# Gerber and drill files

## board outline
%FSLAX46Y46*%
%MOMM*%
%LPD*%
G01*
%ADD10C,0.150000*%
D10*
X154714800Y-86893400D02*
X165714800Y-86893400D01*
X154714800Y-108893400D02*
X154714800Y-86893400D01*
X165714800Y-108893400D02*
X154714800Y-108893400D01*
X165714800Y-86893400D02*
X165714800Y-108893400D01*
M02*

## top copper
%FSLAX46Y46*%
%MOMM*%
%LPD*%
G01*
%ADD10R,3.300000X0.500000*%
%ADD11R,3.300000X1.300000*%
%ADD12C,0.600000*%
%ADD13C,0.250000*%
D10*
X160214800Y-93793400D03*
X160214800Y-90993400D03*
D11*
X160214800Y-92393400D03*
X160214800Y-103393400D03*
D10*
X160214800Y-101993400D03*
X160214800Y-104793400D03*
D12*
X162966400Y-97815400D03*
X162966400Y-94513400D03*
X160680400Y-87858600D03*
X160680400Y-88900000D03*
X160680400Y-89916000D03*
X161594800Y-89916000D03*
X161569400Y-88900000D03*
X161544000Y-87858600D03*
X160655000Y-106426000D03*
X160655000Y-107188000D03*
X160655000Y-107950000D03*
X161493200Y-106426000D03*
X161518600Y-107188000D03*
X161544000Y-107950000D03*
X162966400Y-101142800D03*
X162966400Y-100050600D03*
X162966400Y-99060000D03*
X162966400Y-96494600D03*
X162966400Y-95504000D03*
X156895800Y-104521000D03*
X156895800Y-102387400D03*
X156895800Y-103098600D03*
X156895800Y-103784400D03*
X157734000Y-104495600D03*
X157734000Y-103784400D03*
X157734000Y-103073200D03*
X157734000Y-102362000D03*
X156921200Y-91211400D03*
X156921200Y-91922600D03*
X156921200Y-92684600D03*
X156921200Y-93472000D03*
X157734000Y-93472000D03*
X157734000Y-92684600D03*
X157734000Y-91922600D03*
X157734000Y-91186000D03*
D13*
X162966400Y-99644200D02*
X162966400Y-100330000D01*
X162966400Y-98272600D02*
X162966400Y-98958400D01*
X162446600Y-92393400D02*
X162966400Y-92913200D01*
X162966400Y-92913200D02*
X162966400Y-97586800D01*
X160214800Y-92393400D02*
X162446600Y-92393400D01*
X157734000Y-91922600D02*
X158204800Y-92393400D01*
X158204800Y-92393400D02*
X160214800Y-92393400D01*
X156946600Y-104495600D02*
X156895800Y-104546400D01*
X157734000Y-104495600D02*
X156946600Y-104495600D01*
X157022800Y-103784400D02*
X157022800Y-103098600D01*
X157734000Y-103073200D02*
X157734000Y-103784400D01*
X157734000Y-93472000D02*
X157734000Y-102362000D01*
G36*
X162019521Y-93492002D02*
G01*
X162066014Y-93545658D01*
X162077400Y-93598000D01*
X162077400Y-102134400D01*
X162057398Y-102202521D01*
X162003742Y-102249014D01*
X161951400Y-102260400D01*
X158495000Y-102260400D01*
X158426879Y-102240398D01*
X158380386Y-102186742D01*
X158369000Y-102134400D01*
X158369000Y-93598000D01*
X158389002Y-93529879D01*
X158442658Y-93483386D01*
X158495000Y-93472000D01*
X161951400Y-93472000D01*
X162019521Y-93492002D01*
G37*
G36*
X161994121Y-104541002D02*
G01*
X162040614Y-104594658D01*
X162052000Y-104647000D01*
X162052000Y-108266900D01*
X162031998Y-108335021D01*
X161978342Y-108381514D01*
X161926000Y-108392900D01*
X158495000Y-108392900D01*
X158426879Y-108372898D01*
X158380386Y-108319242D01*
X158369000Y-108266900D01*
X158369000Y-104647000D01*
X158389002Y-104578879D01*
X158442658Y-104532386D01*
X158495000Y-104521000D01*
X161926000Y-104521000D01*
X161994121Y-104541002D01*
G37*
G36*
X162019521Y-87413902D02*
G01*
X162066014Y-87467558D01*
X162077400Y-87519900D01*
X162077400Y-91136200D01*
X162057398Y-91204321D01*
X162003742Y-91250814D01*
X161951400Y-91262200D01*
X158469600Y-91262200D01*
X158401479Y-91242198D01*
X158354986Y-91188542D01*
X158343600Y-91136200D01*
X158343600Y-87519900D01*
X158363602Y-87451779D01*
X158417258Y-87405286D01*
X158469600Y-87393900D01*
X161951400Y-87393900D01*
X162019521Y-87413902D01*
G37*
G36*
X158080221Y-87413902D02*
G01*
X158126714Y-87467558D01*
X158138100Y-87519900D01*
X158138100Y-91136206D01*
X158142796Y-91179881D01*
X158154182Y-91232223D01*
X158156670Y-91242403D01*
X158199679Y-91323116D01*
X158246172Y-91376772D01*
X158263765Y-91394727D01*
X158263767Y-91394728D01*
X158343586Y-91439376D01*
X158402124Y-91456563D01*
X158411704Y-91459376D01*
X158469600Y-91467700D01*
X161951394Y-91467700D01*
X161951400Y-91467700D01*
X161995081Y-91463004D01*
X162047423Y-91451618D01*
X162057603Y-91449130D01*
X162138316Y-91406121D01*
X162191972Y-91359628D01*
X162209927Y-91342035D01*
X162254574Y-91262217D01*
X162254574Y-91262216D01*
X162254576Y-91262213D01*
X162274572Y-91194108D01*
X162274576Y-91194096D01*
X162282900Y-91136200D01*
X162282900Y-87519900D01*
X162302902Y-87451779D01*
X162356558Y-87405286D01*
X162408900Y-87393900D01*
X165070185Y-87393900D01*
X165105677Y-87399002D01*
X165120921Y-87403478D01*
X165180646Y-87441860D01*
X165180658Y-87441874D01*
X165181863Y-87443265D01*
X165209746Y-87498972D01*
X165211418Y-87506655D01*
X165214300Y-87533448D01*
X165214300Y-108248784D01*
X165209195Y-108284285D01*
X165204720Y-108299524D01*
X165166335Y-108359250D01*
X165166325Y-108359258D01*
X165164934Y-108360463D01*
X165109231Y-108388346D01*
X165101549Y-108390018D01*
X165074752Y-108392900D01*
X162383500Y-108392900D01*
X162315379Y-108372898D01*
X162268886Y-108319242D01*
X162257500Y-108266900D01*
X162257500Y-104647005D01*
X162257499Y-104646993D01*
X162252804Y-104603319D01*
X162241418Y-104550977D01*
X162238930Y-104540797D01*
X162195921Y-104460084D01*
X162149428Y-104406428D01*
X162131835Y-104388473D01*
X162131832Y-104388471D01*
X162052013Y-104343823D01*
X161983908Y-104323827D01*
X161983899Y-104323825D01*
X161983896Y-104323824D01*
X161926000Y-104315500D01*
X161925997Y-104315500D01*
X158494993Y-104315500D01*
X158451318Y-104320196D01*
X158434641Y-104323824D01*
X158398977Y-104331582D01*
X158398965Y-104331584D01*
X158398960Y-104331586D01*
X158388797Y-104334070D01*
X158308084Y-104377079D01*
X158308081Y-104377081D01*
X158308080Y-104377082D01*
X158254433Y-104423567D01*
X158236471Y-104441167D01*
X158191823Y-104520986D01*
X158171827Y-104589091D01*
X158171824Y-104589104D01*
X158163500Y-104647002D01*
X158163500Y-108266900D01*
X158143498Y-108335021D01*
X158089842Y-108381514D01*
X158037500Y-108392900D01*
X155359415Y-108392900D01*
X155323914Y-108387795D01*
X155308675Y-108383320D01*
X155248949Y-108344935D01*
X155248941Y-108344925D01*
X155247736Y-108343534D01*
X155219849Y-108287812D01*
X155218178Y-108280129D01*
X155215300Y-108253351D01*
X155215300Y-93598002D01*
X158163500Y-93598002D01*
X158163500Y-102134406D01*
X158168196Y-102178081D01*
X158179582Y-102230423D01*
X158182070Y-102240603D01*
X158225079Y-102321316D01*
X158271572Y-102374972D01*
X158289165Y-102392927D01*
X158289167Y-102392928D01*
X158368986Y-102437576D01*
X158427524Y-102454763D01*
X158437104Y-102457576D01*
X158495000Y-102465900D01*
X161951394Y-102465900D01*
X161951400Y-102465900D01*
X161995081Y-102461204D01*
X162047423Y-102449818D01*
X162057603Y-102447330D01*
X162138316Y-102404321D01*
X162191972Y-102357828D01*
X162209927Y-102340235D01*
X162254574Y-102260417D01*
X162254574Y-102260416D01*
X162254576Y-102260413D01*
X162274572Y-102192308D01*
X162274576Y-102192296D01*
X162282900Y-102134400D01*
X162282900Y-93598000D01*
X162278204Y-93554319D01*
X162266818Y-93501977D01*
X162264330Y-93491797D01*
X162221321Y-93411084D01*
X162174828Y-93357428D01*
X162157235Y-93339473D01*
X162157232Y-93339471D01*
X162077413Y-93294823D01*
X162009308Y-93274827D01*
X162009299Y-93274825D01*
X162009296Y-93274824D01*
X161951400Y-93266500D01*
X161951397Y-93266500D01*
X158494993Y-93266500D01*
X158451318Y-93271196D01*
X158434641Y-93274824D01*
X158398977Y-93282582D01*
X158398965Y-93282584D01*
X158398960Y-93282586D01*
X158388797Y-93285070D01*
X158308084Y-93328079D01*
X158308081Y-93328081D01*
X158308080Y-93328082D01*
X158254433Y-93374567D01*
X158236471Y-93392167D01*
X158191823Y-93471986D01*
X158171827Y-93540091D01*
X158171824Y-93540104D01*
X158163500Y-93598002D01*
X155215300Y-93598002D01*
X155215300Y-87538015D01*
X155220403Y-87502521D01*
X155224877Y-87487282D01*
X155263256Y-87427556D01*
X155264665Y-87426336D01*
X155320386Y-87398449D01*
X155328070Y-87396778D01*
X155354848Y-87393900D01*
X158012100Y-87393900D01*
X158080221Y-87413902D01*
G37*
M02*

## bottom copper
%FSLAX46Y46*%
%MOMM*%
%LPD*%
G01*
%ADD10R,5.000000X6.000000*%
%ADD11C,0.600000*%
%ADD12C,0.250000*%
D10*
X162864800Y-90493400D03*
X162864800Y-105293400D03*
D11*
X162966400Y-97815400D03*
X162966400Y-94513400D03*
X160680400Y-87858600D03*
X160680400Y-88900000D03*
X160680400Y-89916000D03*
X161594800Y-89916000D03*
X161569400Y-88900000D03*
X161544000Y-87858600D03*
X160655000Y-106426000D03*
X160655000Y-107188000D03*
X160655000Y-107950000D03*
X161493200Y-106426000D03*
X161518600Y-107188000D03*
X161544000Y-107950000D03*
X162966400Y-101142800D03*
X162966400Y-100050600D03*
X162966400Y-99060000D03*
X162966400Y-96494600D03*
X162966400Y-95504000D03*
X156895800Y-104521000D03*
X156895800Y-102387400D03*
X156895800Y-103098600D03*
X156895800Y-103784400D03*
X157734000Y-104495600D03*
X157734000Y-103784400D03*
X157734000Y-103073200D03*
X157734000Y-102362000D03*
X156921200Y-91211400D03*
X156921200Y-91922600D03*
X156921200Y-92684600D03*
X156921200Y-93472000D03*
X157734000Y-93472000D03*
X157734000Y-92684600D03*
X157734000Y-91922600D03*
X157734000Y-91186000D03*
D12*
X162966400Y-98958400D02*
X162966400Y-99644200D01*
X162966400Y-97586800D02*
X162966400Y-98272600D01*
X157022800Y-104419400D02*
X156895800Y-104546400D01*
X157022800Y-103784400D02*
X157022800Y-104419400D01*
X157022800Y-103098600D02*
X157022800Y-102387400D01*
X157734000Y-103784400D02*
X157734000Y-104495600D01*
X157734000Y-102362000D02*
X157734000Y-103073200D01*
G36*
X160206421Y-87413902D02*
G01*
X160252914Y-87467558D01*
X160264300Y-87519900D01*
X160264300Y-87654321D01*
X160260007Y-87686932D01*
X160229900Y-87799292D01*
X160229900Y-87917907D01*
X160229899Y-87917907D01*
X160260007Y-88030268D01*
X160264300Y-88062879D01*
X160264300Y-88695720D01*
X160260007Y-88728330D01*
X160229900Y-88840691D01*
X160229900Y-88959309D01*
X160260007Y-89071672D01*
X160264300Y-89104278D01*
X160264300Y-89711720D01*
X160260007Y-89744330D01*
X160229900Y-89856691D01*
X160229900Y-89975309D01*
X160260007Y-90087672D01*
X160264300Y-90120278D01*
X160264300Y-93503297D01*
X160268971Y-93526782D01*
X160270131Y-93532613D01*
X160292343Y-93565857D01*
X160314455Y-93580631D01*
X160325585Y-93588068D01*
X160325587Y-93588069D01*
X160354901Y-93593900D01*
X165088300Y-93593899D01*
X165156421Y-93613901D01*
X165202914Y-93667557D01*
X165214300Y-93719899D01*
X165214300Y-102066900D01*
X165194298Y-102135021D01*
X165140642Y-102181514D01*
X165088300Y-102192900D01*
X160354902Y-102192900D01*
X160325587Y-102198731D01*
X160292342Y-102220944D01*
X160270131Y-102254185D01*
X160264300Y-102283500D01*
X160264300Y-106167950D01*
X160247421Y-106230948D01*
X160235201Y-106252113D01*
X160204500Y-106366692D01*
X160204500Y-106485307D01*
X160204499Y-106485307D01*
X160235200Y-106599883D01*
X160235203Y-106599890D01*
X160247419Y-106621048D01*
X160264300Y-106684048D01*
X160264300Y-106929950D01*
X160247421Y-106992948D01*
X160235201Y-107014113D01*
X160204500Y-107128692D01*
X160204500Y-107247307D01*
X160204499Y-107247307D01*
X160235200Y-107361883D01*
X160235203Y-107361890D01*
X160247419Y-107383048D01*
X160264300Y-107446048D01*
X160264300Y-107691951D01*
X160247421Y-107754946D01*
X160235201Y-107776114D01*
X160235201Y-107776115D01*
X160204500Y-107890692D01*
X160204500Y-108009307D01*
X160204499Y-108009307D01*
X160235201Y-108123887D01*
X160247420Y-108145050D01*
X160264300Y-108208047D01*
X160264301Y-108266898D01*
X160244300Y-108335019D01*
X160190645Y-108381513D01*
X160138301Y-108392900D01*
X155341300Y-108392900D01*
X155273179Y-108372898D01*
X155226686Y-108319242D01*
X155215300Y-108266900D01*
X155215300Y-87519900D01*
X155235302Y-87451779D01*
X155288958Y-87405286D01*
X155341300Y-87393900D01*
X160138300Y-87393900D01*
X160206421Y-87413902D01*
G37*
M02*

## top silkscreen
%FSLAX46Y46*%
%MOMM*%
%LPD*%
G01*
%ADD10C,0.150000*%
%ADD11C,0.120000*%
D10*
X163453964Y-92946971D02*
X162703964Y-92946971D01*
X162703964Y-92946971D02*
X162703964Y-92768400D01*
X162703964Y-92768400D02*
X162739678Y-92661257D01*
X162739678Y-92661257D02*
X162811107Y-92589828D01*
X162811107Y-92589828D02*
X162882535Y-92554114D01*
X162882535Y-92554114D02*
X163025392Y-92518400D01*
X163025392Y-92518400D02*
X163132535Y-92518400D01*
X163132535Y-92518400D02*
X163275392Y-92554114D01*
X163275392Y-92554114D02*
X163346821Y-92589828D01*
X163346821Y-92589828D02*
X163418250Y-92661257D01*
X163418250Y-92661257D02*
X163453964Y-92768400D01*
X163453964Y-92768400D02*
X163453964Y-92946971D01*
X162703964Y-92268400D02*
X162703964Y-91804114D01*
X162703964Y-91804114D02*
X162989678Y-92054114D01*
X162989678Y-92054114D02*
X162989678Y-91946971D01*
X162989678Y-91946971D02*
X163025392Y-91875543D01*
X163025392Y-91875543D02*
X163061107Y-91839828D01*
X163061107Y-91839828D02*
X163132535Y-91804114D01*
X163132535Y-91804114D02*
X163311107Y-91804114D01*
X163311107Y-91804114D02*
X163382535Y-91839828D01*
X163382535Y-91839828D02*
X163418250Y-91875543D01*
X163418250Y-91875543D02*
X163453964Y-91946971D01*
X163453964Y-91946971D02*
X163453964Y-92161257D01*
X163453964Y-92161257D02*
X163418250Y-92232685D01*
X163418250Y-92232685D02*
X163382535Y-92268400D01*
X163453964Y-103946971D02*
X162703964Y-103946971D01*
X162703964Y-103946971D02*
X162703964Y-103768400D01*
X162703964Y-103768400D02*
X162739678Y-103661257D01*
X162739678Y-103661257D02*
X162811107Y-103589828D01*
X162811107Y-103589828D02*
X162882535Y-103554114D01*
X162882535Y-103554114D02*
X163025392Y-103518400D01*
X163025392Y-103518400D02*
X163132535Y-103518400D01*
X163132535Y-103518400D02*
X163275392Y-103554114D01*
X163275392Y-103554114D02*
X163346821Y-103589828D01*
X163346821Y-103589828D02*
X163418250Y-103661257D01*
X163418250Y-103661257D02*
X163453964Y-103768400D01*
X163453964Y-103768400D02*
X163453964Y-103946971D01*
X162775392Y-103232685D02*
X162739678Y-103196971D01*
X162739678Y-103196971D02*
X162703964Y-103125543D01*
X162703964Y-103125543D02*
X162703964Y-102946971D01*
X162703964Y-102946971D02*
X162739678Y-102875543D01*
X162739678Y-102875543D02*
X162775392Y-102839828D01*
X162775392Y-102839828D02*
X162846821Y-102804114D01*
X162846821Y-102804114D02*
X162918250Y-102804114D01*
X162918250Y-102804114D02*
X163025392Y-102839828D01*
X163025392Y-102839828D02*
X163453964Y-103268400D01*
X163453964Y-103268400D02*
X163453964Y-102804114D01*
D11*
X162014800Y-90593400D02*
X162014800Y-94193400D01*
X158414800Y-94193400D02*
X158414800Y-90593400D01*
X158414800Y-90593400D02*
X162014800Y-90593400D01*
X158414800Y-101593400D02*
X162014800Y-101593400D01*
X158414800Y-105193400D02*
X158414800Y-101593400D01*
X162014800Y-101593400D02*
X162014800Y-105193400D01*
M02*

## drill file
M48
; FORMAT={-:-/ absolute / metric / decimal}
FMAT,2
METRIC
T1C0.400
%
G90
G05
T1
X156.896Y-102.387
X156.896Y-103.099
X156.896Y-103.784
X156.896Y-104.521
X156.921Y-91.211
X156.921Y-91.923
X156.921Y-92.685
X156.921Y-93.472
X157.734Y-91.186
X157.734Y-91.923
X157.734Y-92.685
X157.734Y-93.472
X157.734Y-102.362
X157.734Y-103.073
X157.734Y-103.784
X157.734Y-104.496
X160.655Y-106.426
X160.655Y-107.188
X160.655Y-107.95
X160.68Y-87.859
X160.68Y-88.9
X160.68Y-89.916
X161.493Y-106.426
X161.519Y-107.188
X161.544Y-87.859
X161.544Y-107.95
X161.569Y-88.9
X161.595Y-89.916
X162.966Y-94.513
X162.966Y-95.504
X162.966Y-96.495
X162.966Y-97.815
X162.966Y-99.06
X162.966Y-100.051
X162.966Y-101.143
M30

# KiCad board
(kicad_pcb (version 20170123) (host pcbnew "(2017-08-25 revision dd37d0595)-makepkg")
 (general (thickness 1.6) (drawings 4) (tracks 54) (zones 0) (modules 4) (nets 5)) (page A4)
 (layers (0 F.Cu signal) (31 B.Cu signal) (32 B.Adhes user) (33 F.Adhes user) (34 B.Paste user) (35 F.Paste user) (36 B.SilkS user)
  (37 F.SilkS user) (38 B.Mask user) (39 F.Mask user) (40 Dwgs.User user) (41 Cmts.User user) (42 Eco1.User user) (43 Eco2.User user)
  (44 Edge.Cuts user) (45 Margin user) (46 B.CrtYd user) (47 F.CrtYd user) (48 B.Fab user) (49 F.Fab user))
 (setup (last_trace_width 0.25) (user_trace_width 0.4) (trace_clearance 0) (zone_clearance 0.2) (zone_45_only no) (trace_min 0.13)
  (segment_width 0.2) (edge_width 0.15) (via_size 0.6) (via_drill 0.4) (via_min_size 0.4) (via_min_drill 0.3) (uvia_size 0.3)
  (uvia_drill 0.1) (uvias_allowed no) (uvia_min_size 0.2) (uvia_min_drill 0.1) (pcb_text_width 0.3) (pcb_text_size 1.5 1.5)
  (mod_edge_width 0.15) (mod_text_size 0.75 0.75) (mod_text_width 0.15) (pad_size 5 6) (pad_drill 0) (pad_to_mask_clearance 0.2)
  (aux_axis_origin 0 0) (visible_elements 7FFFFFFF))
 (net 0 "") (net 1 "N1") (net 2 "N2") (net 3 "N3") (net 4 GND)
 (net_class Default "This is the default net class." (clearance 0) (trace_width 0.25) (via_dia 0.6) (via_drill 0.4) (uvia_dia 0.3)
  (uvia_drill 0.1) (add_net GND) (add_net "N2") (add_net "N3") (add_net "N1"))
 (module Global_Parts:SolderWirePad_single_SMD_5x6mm (layer B.Cu) (at 162.8648 90.4934)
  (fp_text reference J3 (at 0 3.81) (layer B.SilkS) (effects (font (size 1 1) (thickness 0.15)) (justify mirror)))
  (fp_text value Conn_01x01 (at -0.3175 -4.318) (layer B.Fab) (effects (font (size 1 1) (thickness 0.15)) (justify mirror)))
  (pad 1 smd rect (at 0 0) (size 5 6) (layers B.Cu B.Paste B.Mask) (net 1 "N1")))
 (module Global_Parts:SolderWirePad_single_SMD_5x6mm (layer B.Cu) (at 162.8648 105.2934)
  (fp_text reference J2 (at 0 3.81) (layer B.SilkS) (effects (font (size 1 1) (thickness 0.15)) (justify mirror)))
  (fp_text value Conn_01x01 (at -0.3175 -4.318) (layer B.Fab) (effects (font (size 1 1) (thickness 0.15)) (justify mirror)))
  (pad 1 smd rect (at 0 0) (size 5 6) (layers B.Cu B.Paste B.Mask) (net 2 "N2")))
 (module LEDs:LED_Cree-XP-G (layer F.Cu) (at 160.2148 92.3934 270)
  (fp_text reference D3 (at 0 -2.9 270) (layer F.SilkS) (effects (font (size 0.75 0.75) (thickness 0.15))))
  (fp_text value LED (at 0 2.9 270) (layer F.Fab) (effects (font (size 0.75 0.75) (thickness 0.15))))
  (fp_line (start -1.8 -1.8) (end 1.8 -1.8) (layer F.SilkS) (width 0.12))
  (fp_line (start 1.8 1.8) (end -1.8 1.8) (layer F.SilkS) (width 0.12))
  (fp_line (start -1.8 1.8) (end -1.8 -1.8) (layer F.SilkS) (width 0.12))
  (pad 2 smd rect (at 1.4 0 270) (size 0.5 3.3) (layers F.Cu F.Paste F.Mask) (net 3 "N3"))
  (pad 1 smd rect (at -1.4 0 270) (size 0.5 3.3) (layers F.Cu F.Paste F.Mask) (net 1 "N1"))
  (pad 3 smd rect (at 0 0 270) (size 1.3 3.3) (layers F.Cu F.Mask) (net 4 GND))
  (pad 3 smd rect (at 0 0 270) (size 1.01 0.75) (layers F.Paste))
  (pad 3 smd rect (at 0 1 270) (size 1.01 0.75) (layers F.Paste))
  (pad 3 smd rect (at 0 -1 270) (size 1.01 0.75) (layers F.Paste)))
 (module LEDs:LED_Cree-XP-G (layer F.Cu) (at 160.2148 103.3934 270)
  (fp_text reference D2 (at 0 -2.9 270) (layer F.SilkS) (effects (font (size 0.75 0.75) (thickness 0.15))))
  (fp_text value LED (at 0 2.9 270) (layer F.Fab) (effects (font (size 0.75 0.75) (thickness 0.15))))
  (fp_line (start -1.8 1.8) (end -1.8 -1.8) (layer F.SilkS) (width 0.12))
  (fp_line (start 1.8 1.8) (end -1.8 1.8) (layer F.SilkS) (width 0.12))
  (fp_line (start -1.8 -1.8) (end 1.8 -1.8) (layer F.SilkS) (width 0.12))
  (pad 3 smd rect (at 0 -1 270) (size 1.01 0.75) (layers F.Paste))
  (pad 3 smd rect (at 0 1 270) (size 1.01 0.75) (layers F.Paste))
  (pad 3 smd rect (at 0 0 270) (size 1.01 0.75) (layers F.Paste))
  (pad 3 smd rect (at 0 0 270) (size 1.3 3.3) (layers F.Cu F.Mask) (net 4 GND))
  (pad 1 smd rect (at -1.4 0 270) (size 0.5 3.3) (layers F.Cu F.Paste F.Mask) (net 3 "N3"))
  (pad 2 smd rect (at 1.4 0 270) (size 0.5 3.3) (layers F.Cu F.Paste F.Mask) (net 2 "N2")))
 (gr_line (start 154.7148 86.8934) (end 165.7148 86.8934) (layer Edge.Cuts) (width 0.15))
 (gr_line (start 154.7148 108.8934) (end 154.7148 86.8934) (layer Edge.Cuts) (width 0.15))
 (gr_line (start 165.7148 108.8934) (end 154.7148 108.8934) (layer Edge.Cuts) (width 0.15))
 (gr_line (start 165.7148 86.8934) (end 165.7148 108.8934) (layer Edge.Cuts) (width 0.15))
 (via (at 162.9664 97.8154) (size 0.6) (drill 0.4) (layers F.Cu B.Cu) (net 4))
 (via (at 162.9664 94.5134) (size 0.6) (drill 0.4) (layers F.Cu B.Cu) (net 4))
 (via (at 160.6804 87.8586) (size 0.6) (drill 0.4) (layers F.Cu B.Cu) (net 1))
 (via (at 160.6804 88.9) (size 0.6) (drill 0.4) (layers F.Cu B.Cu) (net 1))
 (via (at 160.6804 89.916) (size 0.6) (drill 0.4) (layers F.Cu B.Cu) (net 1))
 (via (at 161.5948 89.916) (size 0.6) (drill 0.4) (layers F.Cu B.Cu) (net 1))
 (via (at 161.5694 88.9) (size 0.6) (drill 0.4) (layers F.Cu B.Cu) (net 1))
 (via (at 161.544 87.8586) (size 0.6) (drill 0.4) (layers F.Cu B.Cu) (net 1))
 (via (at 160.655 106.426) (size 0.6) (drill 0.4) (layers F.Cu B.Cu) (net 2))
 (via (at 160.655 107.188) (size 0.6) (drill 0.4) (layers F.Cu B.Cu) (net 2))
 (via (at 160.655 107.95) (size 0.6) (drill 0.4) (layers F.Cu B.Cu) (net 2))
 (via (at 161.4932 106.426) (size 0.6) (drill 0.4) (layers F.Cu B.Cu) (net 2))
 (via (at 161.5186 107.188) (size 0.6) (drill 0.4) (layers F.Cu B.Cu) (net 2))
 (via (at 161.544 107.95) (size 0.6) (drill 0.4) (layers F.Cu B.Cu) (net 2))
 (segment (start 162.9664 99.6442) (end 162.9664 100.33) (width 0.25) (layer F.Cu) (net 4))
 (via (at 162.9664 101.1428) (size 0.6) (drill 0.4) (layers F.Cu B.Cu) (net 4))
 (segment (start 162.9664 98.9584) (end 162.9664 99.6442) (width 0.25) (layer B.Cu) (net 4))
 (via (at 162.9664 100.0506) (size 0.6) (drill 0.4) (layers F.Cu B.Cu) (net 4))
 (segment (start 162.9664 98.2726) (end 162.9664 98.9584) (width 0.25) (layer F.Cu) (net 4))
 (via (at 162.9664 99.06) (size 0.6) (drill 0.4) (layers F.Cu B.Cu) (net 4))
 (segment (start 162.9664 97.5868) (end 162.9664 98.2726) (width 0.25) (layer B.Cu) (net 4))
 (via (at 162.9664 96.4946) (size 0.6) (drill 0.4) (layers F.Cu B.Cu) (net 4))
 (segment (start 162.4466 92.3934) (end 162.9664 92.9132) (width 0.25) (layer F.Cu) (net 4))
 (segment (start 162.9664 92.9132) (end 162.9664 97.5868) (width 0.25) (layer F.Cu) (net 4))
 (via (at 162.9664 95.504) (size 0.6) (drill 0.4) (layers F.Cu B.Cu) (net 4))
 (segment (start 160.2148 92.3934) (end 162.4466 92.3934) (width 0.25) (layer F.Cu) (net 4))
 (segment (start 157.734 91.9226) (end 158.2048 92.3934) (width 0.25) (layer F.Cu) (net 4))
 (segment (start 158.2048 92.3934) (end 160.2148 92.3934) (width 0.25) (layer F.Cu) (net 4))
 (segment (start 156.9466 104.4956) (end 156.8958 104.5464) (width 0.25) (layer F.Cu) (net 4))
 (segment (start 157.0228 104.4194) (end 156.8958 104.5464) (width 0.25) (layer B.Cu) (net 4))
 (segment (start 157.0228 103.7844) (end 157.0228 104.4194) (width 0.25) (layer B.Cu) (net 4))
 (segment (start 157.734 104.4956) (end 156.9466 104.4956) (width 0.25) (layer F.Cu) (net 4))
 (via (at 156.8958 104.521) (size 0.6) (drill 0.4) (layers F.Cu B.Cu) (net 4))
 (segment (start 157.0228 103.0986) (end 157.0228 102.3874) (width 0.25) (layer B.Cu) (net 4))
 (via (at 156.8958 102.3874) (size 0.6) (drill 0.4) (layers F.Cu B.Cu) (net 4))
 (segment (start 157.0228 103.7844) (end 157.0228 103.0986) (width 0.25) (layer F.Cu) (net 4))
 (via (at 156.8958 103.0986) (size 0.6) (drill 0.4) (layers F.Cu B.Cu) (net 4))
 (via (at 156.8958 103.7844) (size 0.6) (drill 0.4) (layers F.Cu B.Cu) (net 4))
 (segment (start 157.734 103.7844) (end 157.734 104.4956) (width 0.25) (layer B.Cu) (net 4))
 (via (at 157.734 104.4956) (size 0.6) (drill 0.4) (layers F.Cu B.Cu) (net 4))
 (segment (start 157.734 103.0732) (end 157.734 103.7844) (width 0.25) (layer F.Cu) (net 4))
 (via (at 157.734 103.7844) (size 0.6) (drill 0.4) (layers F.Cu B.Cu) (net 4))
 (segment (start 157.734 102.362) (end 157.734 103.0732) (width 0.25) (layer B.Cu) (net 4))
 (via (at 157.734 103.0732) (size 0.6) (drill 0.4) (layers F.Cu B.Cu) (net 4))
 (segment (start 157.734 93.472) (end 157.734 102.362) (width 0.25) (layer F.Cu) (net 4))
 (via (at 157.734 102.362) (size 0.6) (drill 0.4) (layers F.Cu B.Cu) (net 4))
 (via (at 156.9212 91.2114) (size 0.6) (drill 0.4) (layers F.Cu B.Cu) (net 4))
 (via (at 156.9212 91.9226) (size 0.6) (drill 0.4) (layers F.Cu B.Cu) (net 4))
 (via (at 156.9212 92.6846) (size 0.6) (drill 0.4) (layers F.Cu B.Cu) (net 4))
 (via (at 156.9212 93.472) (size 0.6) (drill 0.4) (layers F.Cu B.Cu) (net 4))
 (via (at 157.734 93.472) (size 0.6) (drill 0.4) (layers F.Cu B.Cu) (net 4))
 (via (at 157.734 92.6846) (size 0.6) (drill 0.4) (layers F.Cu B.Cu) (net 4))
 (via (at 157.734 91.9226) (size 0.6) (drill 0.4) (layers F.Cu B.Cu) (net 4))
 (via (at 157.734 91.186) (size 0.6) (drill 0.4) (layers F.Cu B.Cu) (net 4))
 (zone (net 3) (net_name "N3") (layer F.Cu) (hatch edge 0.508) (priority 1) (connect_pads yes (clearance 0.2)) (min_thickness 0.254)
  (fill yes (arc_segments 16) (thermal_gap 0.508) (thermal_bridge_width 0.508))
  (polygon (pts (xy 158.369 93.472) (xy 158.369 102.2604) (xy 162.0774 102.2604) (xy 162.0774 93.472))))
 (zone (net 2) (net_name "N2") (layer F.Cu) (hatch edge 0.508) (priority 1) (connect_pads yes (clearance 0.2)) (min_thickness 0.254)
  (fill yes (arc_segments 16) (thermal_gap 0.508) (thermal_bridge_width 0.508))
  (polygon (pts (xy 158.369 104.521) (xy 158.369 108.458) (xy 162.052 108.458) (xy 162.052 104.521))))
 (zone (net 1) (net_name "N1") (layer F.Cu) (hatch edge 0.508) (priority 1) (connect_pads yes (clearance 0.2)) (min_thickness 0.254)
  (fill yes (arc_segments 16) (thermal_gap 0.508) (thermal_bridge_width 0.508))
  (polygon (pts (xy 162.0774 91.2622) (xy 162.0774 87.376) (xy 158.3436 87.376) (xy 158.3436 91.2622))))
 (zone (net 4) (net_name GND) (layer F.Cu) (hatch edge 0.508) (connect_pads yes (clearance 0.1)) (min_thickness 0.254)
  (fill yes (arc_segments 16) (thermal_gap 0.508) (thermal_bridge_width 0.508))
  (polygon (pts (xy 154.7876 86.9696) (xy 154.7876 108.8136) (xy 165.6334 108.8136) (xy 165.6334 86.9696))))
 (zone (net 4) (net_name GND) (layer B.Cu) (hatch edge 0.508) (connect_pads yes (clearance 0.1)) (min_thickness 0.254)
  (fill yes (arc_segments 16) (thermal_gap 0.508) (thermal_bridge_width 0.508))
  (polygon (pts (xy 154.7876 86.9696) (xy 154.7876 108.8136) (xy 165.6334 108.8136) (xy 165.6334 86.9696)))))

